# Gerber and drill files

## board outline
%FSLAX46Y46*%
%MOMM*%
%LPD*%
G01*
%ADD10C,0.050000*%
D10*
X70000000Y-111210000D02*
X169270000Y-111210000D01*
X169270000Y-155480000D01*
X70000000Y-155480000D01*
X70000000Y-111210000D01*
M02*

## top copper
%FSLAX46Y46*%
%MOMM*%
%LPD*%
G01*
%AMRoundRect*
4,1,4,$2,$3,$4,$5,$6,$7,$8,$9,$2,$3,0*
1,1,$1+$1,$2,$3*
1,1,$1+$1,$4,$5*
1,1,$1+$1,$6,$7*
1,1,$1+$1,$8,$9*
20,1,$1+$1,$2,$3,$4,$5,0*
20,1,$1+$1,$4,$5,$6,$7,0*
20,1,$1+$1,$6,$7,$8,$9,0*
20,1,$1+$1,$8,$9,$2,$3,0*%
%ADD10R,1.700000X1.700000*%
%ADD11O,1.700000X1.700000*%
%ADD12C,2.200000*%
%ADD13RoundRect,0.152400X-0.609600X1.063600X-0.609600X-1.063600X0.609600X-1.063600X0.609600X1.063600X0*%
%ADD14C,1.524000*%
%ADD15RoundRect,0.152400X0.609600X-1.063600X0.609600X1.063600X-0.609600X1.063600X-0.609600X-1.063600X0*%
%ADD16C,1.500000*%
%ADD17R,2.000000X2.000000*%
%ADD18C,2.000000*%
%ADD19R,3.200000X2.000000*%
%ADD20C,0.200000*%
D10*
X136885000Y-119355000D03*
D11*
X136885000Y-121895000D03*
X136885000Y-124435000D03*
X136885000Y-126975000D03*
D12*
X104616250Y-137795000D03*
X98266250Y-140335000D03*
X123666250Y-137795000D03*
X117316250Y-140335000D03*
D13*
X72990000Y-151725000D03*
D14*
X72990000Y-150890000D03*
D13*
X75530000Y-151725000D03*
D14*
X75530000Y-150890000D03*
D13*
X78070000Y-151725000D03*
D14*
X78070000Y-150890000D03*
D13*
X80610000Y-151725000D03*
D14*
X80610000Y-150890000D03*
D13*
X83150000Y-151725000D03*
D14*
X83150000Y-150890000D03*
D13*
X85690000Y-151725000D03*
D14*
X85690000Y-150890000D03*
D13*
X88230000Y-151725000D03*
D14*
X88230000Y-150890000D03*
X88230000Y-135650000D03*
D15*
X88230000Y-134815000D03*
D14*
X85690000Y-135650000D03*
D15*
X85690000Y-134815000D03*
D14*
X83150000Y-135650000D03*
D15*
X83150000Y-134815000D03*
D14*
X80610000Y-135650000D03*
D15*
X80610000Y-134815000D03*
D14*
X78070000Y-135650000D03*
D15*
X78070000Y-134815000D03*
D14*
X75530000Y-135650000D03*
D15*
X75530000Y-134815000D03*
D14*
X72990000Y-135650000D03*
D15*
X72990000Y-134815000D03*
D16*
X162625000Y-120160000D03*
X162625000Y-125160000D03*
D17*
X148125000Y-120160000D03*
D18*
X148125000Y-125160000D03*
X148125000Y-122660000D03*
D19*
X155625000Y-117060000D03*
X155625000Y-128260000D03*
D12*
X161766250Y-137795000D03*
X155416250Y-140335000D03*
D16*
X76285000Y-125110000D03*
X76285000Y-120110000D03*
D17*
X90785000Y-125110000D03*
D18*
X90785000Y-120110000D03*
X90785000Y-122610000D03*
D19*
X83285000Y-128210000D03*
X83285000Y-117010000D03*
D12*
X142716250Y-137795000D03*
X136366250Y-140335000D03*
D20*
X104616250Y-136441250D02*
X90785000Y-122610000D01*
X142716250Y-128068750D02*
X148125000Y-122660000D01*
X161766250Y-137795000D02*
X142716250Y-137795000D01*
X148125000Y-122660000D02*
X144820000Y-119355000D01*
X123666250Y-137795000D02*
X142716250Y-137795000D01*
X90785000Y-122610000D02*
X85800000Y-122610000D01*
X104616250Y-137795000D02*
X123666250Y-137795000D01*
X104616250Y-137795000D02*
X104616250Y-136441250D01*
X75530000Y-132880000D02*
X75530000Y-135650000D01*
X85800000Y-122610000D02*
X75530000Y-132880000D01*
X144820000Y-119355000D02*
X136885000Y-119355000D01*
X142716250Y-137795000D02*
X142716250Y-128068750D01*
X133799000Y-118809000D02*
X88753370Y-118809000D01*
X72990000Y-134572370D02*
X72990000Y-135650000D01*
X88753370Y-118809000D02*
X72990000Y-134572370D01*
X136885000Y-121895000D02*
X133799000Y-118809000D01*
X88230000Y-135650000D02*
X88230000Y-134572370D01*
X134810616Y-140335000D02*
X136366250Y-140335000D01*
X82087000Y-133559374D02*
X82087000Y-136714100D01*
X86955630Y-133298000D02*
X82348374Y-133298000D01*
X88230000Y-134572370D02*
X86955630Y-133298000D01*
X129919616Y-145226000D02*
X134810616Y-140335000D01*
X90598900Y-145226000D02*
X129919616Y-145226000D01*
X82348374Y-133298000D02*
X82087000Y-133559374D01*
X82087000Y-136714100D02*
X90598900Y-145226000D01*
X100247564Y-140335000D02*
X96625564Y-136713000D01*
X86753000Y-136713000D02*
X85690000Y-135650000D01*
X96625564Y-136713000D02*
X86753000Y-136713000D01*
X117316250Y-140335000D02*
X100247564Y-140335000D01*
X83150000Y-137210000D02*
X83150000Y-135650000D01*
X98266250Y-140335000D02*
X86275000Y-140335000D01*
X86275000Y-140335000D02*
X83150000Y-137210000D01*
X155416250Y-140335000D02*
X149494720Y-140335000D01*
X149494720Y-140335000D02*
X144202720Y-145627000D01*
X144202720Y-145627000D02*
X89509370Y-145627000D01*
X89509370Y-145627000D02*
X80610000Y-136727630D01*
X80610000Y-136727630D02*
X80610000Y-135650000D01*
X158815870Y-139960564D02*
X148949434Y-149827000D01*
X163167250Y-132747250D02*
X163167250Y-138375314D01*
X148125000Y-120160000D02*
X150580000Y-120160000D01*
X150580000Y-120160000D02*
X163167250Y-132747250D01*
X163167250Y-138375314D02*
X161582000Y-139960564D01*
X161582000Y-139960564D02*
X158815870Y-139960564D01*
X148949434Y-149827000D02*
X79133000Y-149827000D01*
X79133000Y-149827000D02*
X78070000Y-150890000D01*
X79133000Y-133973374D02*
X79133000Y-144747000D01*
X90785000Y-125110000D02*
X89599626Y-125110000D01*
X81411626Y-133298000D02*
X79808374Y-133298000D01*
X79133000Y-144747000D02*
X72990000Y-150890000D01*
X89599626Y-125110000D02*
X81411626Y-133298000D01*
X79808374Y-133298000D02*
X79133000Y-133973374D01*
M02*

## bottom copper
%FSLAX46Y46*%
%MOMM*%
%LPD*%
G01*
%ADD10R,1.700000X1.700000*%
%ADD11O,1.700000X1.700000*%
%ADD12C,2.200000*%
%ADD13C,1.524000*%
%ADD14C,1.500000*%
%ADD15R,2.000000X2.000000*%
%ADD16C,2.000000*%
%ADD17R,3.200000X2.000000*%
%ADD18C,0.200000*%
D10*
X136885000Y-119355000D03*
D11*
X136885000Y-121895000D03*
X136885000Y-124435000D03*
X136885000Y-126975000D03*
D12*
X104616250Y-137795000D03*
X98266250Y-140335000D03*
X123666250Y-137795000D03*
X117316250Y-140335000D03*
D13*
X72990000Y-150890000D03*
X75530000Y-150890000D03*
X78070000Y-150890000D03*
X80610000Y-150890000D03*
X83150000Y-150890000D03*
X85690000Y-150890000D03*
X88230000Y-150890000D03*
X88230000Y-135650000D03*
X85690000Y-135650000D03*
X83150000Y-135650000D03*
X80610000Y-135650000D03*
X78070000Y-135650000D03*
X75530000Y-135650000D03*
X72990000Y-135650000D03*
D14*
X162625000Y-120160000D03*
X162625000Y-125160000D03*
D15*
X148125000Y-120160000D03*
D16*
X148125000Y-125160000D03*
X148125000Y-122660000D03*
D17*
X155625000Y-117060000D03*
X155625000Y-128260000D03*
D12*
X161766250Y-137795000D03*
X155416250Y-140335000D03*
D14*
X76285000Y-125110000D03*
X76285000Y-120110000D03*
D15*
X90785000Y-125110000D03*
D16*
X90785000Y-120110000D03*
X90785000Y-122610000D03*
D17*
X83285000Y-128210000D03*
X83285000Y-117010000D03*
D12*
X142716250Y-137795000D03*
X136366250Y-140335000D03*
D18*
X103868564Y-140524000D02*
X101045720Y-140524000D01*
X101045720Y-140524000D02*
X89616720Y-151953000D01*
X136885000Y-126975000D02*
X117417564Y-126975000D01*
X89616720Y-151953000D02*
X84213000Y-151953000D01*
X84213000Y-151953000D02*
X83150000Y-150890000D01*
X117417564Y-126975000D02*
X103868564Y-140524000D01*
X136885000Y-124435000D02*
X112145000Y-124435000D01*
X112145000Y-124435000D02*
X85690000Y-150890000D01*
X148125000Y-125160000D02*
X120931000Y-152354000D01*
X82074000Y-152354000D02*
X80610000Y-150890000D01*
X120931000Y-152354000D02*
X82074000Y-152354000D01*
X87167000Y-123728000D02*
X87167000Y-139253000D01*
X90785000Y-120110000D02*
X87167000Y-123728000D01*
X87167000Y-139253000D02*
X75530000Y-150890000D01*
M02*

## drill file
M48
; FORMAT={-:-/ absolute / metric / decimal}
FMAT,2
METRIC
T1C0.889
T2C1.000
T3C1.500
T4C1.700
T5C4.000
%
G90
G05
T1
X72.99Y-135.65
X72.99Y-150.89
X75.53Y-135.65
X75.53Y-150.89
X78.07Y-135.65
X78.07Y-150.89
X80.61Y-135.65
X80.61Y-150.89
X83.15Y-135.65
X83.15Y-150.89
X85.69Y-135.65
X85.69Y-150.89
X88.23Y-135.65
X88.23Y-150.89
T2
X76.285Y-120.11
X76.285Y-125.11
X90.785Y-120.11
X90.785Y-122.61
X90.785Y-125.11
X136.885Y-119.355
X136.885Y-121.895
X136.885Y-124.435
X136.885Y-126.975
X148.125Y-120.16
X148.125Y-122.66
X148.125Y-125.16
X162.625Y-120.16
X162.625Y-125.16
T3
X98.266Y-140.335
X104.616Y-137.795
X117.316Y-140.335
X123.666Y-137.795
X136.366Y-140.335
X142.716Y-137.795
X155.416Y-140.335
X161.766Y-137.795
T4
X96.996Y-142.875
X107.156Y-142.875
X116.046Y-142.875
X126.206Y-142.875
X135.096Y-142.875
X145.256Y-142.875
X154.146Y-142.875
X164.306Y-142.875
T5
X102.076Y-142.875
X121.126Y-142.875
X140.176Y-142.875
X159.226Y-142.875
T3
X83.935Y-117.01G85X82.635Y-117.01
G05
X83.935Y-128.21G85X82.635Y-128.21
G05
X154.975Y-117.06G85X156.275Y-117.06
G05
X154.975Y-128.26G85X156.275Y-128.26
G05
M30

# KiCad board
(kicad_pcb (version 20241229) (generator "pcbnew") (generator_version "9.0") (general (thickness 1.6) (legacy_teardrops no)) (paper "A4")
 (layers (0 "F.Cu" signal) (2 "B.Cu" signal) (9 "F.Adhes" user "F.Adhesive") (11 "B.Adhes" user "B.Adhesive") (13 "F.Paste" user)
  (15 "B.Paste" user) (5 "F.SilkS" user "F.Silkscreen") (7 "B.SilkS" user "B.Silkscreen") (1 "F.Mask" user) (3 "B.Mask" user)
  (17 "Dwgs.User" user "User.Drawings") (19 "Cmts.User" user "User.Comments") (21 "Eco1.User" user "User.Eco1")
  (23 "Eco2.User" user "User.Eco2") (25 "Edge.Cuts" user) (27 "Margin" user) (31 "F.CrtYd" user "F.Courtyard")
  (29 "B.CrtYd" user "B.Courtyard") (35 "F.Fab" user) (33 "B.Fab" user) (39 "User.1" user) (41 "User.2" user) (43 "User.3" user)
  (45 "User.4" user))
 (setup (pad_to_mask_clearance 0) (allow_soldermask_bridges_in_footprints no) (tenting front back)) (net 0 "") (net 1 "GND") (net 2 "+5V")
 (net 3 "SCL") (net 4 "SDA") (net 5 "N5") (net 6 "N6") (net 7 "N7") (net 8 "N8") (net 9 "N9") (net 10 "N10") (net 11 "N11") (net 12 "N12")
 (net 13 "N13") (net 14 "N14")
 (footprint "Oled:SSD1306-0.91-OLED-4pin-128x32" (layer "F.Cu") (at 100.385 117.165)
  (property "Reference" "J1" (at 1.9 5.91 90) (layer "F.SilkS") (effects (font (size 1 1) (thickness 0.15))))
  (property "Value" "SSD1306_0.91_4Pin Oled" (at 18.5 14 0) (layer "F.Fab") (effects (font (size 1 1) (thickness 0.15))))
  (pad "1" thru_hole rect (at 36.5 2.19) (size 1.7 1.7) (drill 1) (layers "*.Cu" "*.Mask") (remove_unused_layers no) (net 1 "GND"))
  (pad "2" thru_hole oval (at 36.5 4.73) (size 1.7 1.7) (drill 1) (layers "*.Cu" "*.Mask") (remove_unused_layers no) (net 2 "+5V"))
  (pad "3" thru_hole oval (at 36.5 7.27) (size 1.7 1.7) (drill 1) (layers "*.Cu" "*.Mask") (remove_unused_layers no) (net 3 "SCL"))
  (pad "4" thru_hole oval (at 36.5 9.81) (size 1.7 1.7) (drill 1) (layers "*.Cu" "*.Mask") (remove_unused_layers no) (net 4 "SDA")))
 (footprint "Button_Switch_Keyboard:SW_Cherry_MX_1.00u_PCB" (layer "F.Cu") (at 104.61625 137.795)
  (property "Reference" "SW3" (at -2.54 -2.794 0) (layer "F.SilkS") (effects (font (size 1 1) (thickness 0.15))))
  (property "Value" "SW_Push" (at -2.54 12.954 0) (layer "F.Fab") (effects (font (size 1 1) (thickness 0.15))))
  (pad "" np_thru_hole circle (at -7.62 5.08) (size 1.7 1.7) (drill 1.7) (layers "*.Cu" "*.Mask"))
  (pad "" np_thru_hole circle (at -2.54 5.08) (size 4 4) (drill 4) (layers "*.Cu" "*.Mask"))
  (pad "" np_thru_hole circle (at 2.54 5.08) (size 1.7 1.7) (drill 1.7) (layers "*.Cu" "*.Mask"))
  (pad "1" thru_hole circle (at 0 0) (size 2.2 2.2) (drill 1.5) (layers "*.Cu" "*.Mask") (remove_unused_layers no) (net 1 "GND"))
  (pad "2" thru_hole circle (at -6.35 2.54) (size 2.2 2.2) (drill 1.5) (layers "*.Cu" "*.Mask") (remove_unused_layers no) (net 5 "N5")))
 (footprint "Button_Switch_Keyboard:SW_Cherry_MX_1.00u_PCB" (layer "F.Cu") (at 123.66625 137.795)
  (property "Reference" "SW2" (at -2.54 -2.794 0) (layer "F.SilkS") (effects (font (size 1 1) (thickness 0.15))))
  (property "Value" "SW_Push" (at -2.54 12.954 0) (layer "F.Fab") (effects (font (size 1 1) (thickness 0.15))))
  (pad "" np_thru_hole circle (at -7.62 5.08) (size 1.7 1.7) (drill 1.7) (layers "*.Cu" "*.Mask"))
  (pad "" np_thru_hole circle (at -2.54 5.08) (size 4 4) (drill 4) (layers "*.Cu" "*.Mask"))
  (pad "" np_thru_hole circle (at 2.54 5.08) (size 1.7 1.7) (drill 1.7) (layers "*.Cu" "*.Mask"))
  (pad "1" thru_hole circle (at 0 0) (size 2.2 2.2) (drill 1.5) (layers "*.Cu" "*.Mask") (remove_unused_layers no) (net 1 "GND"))
  (pad "2" thru_hole circle (at -6.35 2.54) (size 2.2 2.2) (drill 1.5) (layers "*.Cu" "*.Mask") (remove_unused_layers no) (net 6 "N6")))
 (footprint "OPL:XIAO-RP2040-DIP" (layer "F.Cu") (at 80.61 143.27 90)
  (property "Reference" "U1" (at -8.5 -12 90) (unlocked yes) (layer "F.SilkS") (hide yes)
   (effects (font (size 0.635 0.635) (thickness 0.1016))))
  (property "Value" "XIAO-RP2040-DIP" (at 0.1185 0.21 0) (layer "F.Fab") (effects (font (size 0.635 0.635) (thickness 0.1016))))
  (pad "1" smd roundrect (at -8.455 -7.62 270) (size 2.432 1.524) (layers "F.Cu" "F.Mask") (roundrect_rratio 0.1) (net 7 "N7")
   (thermal_bridge_angle 45))
  (pad "1" thru_hole circle (at -7.62 -7.62 270) (size 1.524 1.524) (drill 0.889) (layers "*.Cu" "*.Mask") (remove_unused_layers no)
   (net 7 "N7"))
  (pad "2" smd roundrect (at -8.455 -5.08 270) (size 2.432 1.524) (layers "F.Cu" "F.Mask") (roundrect_rratio 0.1) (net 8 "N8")
   (thermal_bridge_angle 45))
  (pad "2" thru_hole circle (at -7.62 -5.08 270) (size 1.524 1.524) (drill 0.889) (layers "*.Cu" "*.Mask") (remove_unused_layers no)
   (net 8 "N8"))
  (pad "3" smd roundrect (at -8.455 -2.54 270) (size 2.432 1.524) (layers "F.Cu" "F.Mask") (roundrect_rratio 0.1) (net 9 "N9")
   (thermal_bridge_angle 45))
  (pad "3" thru_hole circle (at -7.62 -2.54 270) (size 1.524 1.524) (drill 0.889) (layers "*.Cu" "*.Mask") (remove_unused_layers no)
   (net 9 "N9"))
  (pad "4" smd roundrect (at -8.455 0 270) (size 2.432 1.524) (layers "F.Cu" "F.Mask") (roundrect_rratio 0.1) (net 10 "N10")
   (thermal_bridge_angle 45))
  (pad "4" thru_hole circle (at -7.62 0 270) (size 1.524 1.524) (drill 0.889) (layers "*.Cu" "*.Mask") (remove_unused_layers no)
   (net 10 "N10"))
  (pad "5" smd roundrect (at -8.455 2.54 270) (size 2.432 1.524) (layers "F.Cu" "F.Mask") (roundrect_rratio 0.1) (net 4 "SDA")
   (thermal_bridge_angle 45))
  (pad "5" thru_hole circle (at -7.62 2.54 270) (size 1.524 1.524) (drill 0.889) (layers "*.Cu" "*.Mask") (remove_unused_layers no)
   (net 4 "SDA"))
  (pad "6" smd roundrect (at -8.455 5.08 270) (size 2.432 1.524) (layers "F.Cu" "F.Mask") (roundrect_rratio 0.1) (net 3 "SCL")
   (thermal_bridge_angle 45))
  (pad "6" thru_hole circle (at -7.62 5.08 270) (size 1.524 1.524) (drill 0.889) (layers "*.Cu" "*.Mask") (remove_unused_layers no)
   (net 3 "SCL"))
  (pad "7" smd roundrect (at -8.455 7.62 270) (size 2.432 1.524) (layers "F.Cu" "F.Mask") (roundrect_rratio 0.1) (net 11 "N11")
   (thermal_bridge_angle 45))
  (pad "7" thru_hole circle (at -7.62 7.62 270) (size 1.524 1.524) (drill 0.889) (layers "*.Cu" "*.Mask") (remove_unused_layers no)
   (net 11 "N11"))
  (pad "8" thru_hole circle (at 7.62 7.62 90) (size 1.524 1.524) (drill 0.889) (layers "*.Cu" "*.Mask") (remove_unused_layers no)
   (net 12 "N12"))
  (pad "8" smd roundrect (at 8.455 7.62 90) (size 2.432 1.524) (layers "F.Cu" "F.Mask") (roundrect_rratio 0.1) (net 12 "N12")
   (thermal_bridge_angle 45))
  (pad "9" thru_hole circle (at 7.62 5.08 90) (size 1.524 1.524) (drill 0.889) (layers "*.Cu" "*.Mask") (remove_unused_layers no)
   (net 6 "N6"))
  (pad "9" smd roundrect (at 8.455 5.08 90) (size 2.432 1.524) (layers "F.Cu" "F.Mask") (roundrect_rratio 0.1) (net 6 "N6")
   (thermal_bridge_angle 45))
  (pad "10" thru_hole circle (at 7.62 2.54 90) (size 1.524 1.524) (drill 0.889) (layers "*.Cu" "*.Mask") (remove_unused_layers no)
   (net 5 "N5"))
  (pad "10" smd roundrect (at 8.455 2.54 90) (size 2.432 1.524) (layers "F.Cu" "F.Mask") (roundrect_rratio 0.1) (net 5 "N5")
   (thermal_bridge_angle 45))
  (pad "11" thru_hole circle (at 7.62 0 90) (size 1.524 1.524) (drill 0.889) (layers "*.Cu" "*.Mask") (remove_unused_layers no)
   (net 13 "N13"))
  (pad "11" smd roundrect (at 8.455 0 90) (size 2.432 1.524) (layers "F.Cu" "F.Mask") (roundrect_rratio 0.1) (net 13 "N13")
   (thermal_bridge_angle 45))
  (pad "12" thru_hole circle (at 7.62 -2.54 90) (size 1.524 1.524) (drill 0.889) (layers "*.Cu" "*.Mask") (remove_unused_layers no)
   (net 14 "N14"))
  (pad "12" smd roundrect (at 8.455 -2.54 90) (size 2.432 1.524) (layers "F.Cu" "F.Mask") (roundrect_rratio 0.1) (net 14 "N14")
   (thermal_bridge_angle 45))
  (pad "13" thru_hole circle (at 7.62 -5.08 90) (size 1.524 1.524) (drill 0.889) (layers "*.Cu" "*.Mask") (remove_unused_layers no)
   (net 1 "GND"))
  (pad "13" smd roundrect (at 8.455 -5.08 90) (size 2.432 1.524) (layers "F.Cu" "F.Mask") (roundrect_rratio 0.1) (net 1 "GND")
   (thermal_bridge_angle 45))
  (pad "14" thru_hole circle (at 7.62 -7.62 90) (size 1.524 1.524) (drill 0.889) (layers "*.Cu" "*.Mask") (remove_unused_layers no)
   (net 2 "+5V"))
  (pad "14" smd roundrect (at 8.455 -7.62 90) (size 2.432 1.524) (layers "F.Cu" "F.Mask") (roundrect_rratio 0.1) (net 2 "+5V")
   (thermal_bridge_angle 45)))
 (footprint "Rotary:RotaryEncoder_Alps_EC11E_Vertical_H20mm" (layer "F.Cu") (at 148.125 120.16)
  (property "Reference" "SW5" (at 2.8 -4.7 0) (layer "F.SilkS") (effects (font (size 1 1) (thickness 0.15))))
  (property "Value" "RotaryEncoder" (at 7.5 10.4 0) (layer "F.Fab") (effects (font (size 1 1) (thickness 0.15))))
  (pad "" thru_hole circle (at 14.5 0) (size 1.5 1.5) (drill 1) (layers "*.Cu" "*.Mask") (remove_unused_layers no))
  (pad "" thru_hole circle (at 14.5 5) (size 1.5 1.5) (drill 1) (layers "*.Cu" "*.Mask") (remove_unused_layers no))
  (pad "A" thru_hole rect (at 0 0) (size 2 2) (drill 1) (layers "*.Cu" "*.Mask") (remove_unused_layers no) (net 9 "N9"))
  (pad "B" thru_hole circle (at 0 5) (size 2 2) (drill 1) (layers "*.Cu" "*.Mask") (remove_unused_layers no) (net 10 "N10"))
  (pad "C" thru_hole circle (at 0 2.5) (size 2 2) (drill 1) (layers "*.Cu" "*.Mask") (remove_unused_layers no) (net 1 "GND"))
  (pad "MP" thru_hole rect (at 7.5 -3.1) (size 3.2 2) (drill oval 2.8 1.5) (layers "*.Cu" "*.Mask") (remove_unused_layers no))
  (pad "MP" thru_hole rect (at 7.5 8.1) (size 3.2 2) (drill oval 2.8 1.5) (layers "*.Cu" "*.Mask") (remove_unused_layers no)))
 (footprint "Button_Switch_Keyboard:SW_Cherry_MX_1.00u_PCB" (layer "F.Cu") (at 161.76625 137.795)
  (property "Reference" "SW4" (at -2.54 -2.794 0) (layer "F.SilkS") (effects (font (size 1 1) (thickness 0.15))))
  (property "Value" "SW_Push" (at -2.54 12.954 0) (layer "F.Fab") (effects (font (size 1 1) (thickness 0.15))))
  (pad "" np_thru_hole circle (at -7.62 5.08) (size 1.7 1.7) (drill 1.7) (layers "*.Cu" "*.Mask"))
  (pad "" np_thru_hole circle (at -2.54 5.08) (size 4 4) (drill 4) (layers "*.Cu" "*.Mask"))
  (pad "" np_thru_hole circle (at 2.54 5.08) (size 1.7 1.7) (drill 1.7) (layers "*.Cu" "*.Mask"))
  (pad "1" thru_hole circle (at 0 0) (size 2.2 2.2) (drill 1.5) (layers "*.Cu" "*.Mask") (remove_unused_layers no) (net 1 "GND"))
  (pad "2" thru_hole circle (at -6.35 2.54) (size 2.2 2.2) (drill 1.5) (layers "*.Cu" "*.Mask") (remove_unused_layers no) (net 13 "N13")))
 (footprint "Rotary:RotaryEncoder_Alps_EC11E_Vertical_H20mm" (layer "F.Cu") (at 90.785 125.11 180)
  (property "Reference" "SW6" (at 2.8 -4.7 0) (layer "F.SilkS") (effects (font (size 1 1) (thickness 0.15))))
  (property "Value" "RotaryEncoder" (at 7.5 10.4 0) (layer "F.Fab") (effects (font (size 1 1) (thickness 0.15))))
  (pad "" thru_hole circle (at 14.5 0 180) (size 1.5 1.5) (drill 1) (layers "*.Cu" "*.Mask") (remove_unused_layers no))
  (pad "" thru_hole circle (at 14.5 5 180) (size 1.5 1.5) (drill 1) (layers "*.Cu" "*.Mask") (remove_unused_layers no))
  (pad "A" thru_hole rect (at 0 0 180) (size 2 2) (drill 1) (layers "*.Cu" "*.Mask") (remove_unused_layers no) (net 7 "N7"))
  (pad "B" thru_hole circle (at 0 5 180) (size 2 2) (drill 1) (layers "*.Cu" "*.Mask") (remove_unused_layers no) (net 8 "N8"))
  (pad "C" thru_hole circle (at 0 2.5 180) (size 2 2) (drill 1) (layers "*.Cu" "*.Mask") (remove_unused_layers no) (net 1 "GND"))
  (pad "MP" thru_hole rect (at 7.5 -3.1 180) (size 3.2 2) (drill oval 2.8 1.5) (layers "*.Cu" "*.Mask") (remove_unused_layers no))
  (pad "MP" thru_hole rect (at 7.5 8.1 180) (size 3.2 2) (drill oval 2.8 1.5) (layers "*.Cu" "*.Mask") (remove_unused_layers no)))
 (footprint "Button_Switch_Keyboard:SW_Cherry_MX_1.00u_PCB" (layer "F.Cu") (at 142.71625 137.795)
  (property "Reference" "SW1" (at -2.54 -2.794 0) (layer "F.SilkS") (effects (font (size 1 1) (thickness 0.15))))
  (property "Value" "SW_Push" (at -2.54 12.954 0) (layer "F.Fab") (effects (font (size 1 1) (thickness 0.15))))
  (pad "" np_thru_hole circle (at -7.62 5.08) (size 1.7 1.7) (drill 1.7) (layers "*.Cu" "*.Mask"))
  (pad "" np_thru_hole circle (at -2.54 5.08) (size 4 4) (drill 4) (layers "*.Cu" "*.Mask"))
  (pad "" np_thru_hole circle (at 2.54 5.08) (size 1.7 1.7) (drill 1.7) (layers "*.Cu" "*.Mask"))
  (pad "1" thru_hole circle (at 0 0) (size 2.2 2.2) (drill 1.5) (layers "*.Cu" "*.Mask") (remove_unused_layers no) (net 1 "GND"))
  (pad "2" thru_hole circle (at -6.35 2.54) (size 2.2 2.2) (drill 1.5) (layers "*.Cu" "*.Mask") (remove_unused_layers no) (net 12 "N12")))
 (gr_rect (start 70 111.21) (end 169.27 155.48) (stroke (width 0.05) (type default)) (fill no) (layer "Edge.Cuts"))
 (segment (start 103.868564 140.524) (end 101.04572 140.524) (width 0.2) (layer "B.Cu") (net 4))
 (segment (start 101.04572 140.524) (end 89.61672 151.953) (width 0.2) (layer "B.Cu") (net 4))
 (segment (start 136.885 126.975) (end 117.417564 126.975) (width 0.2) (layer "B.Cu") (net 4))
 (segment (start 89.61672 151.953) (end 84.213 151.953) (width 0.2) (layer "B.Cu") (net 4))
 (segment (start 84.213 151.953) (end 83.15 150.89) (width 0.2) (layer "B.Cu") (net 4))
 (segment (start 117.417564 126.975) (end 103.868564 140.524) (width 0.2) (layer "B.Cu") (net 4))
 (segment (start 104.61625 136.44125) (end 90.785 122.61) (width 0.2) (layer "F.Cu") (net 1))
 (segment (start 142.71625 128.06875) (end 148.125 122.66) (width 0.2) (layer "F.Cu") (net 1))
 (segment (start 161.76625 137.795) (end 142.71625 137.795) (width 0.2) (layer "F.Cu") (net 1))
 (segment (start 148.125 122.66) (end 144.82 119.355) (width 0.2) (layer "F.Cu") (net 1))
 (segment (start 123.66625 137.795) (end 142.71625 137.795) (width 0.2) (layer "F.Cu") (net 1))
 (segment (start 90.785 122.61) (end 85.8 122.61) (width 0.2) (layer "F.Cu") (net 1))
 (segment (start 104.61625 137.795) (end 123.66625 137.795) (width 0.2) (layer "F.Cu") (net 1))
 (segment (start 104.61625 137.795) (end 104.61625 136.44125) (width 0.2) (layer "F.Cu") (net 1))
 (segment (start 75.53 132.88) (end 75.53 135.65) (width 0.2) (layer "F.Cu") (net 1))
 (segment (start 85.8 122.61) (end 75.53 132.88) (width 0.2) (layer "F.Cu") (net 1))
 (segment (start 144.82 119.355) (end 136.885 119.355) (width 0.2) (layer "F.Cu") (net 1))
 (segment (start 142.71625 137.795) (end 142.71625 128.06875) (width 0.2) (layer "F.Cu") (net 1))
 (segment (start 133.799 118.809) (end 88.75337 118.809) (width 0.2) (layer "F.Cu") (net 2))
 (segment (start 72.99 134.57237) (end 72.99 135.65) (width 0.2) (layer "F.Cu") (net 2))
 (segment (start 88.75337 118.809) (end 72.99 134.57237) (width 0.2) (layer "F.Cu") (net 2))
 (segment (start 136.885 121.895) (end 133.799 118.809) (width 0.2) (layer "F.Cu") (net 2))
 (segment (start 136.885 124.435) (end 112.145 124.435) (width 0.2) (layer "B.Cu") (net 3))
 (segment (start 112.145 124.435) (end 85.69 150.89) (width 0.2) (layer "B.Cu") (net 3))
 (segment (start 88.23 135.65) (end 88.23 134.57237) (width 0.2) (layer "F.Cu") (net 12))
 (segment (start 134.810616 140.335) (end 136.36625 140.335) (width 0.2) (layer "F.Cu") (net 12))
 (segment (start 82.087 133.559374) (end 82.087 136.7141) (width 0.2) (layer "F.Cu") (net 12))
 (segment (start 86.95563 133.298) (end 82.348374 133.298) (width 0.2) (layer "F.Cu") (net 12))
 (segment (start 88.23 134.57237) (end 86.95563 133.298) (width 0.2) (layer "F.Cu") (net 12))
 (segment (start 129.919616 145.226) (end 134.810616 140.335) (width 0.2) (layer "F.Cu") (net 12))
 (segment (start 90.5989 145.226) (end 129.919616 145.226) (width 0.2) (layer "F.Cu") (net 12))
 (segment (start 82.348374 133.298) (end 82.087 133.559374) (width 0.2) (layer "F.Cu") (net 12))
 (segment (start 82.087 136.7141) (end 90.5989 145.226) (width 0.2) (layer "F.Cu") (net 12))
 (segment (start 100.247564 140.335) (end 96.625564 136.713) (width 0.2) (layer "F.Cu") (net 6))
 (segment (start 86.753 136.713) (end 85.69 135.65) (width 0.2) (layer "F.Cu") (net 6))
 (segment (start 96.625564 136.713) (end 86.753 136.713) (width 0.2) (layer "F.Cu") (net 6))
 (segment (start 117.31625 140.335) (end 100.247564 140.335) (width 0.2) (layer "F.Cu") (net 6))
 (segment (start 83.15 137.21) (end 83.15 135.65) (width 0.2) (layer "F.Cu") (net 5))
 (segment (start 98.26625 140.335) (end 86.275 140.335) (width 0.2) (layer "F.Cu") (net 5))
 (segment (start 86.275 140.335) (end 83.15 137.21) (width 0.2) (layer "F.Cu") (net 5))
 (segment (start 155.41625 140.335) (end 149.49472 140.335) (width 0.2) (layer "F.Cu") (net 13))
 (segment (start 149.49472 140.335) (end 144.20272 145.627) (width 0.2) (layer "F.Cu") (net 13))
 (segment (start 144.20272 145.627) (end 89.50937 145.627) (width 0.2) (layer "F.Cu") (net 13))
 (segment (start 89.50937 145.627) (end 80.61 136.72763) (width 0.2) (layer "F.Cu") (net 13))
 (segment (start 80.61 136.72763) (end 80.61 135.65) (width 0.2) (layer "F.Cu") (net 13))
 (segment (start 148.125 125.16) (end 120.931 152.354) (width 0.2) (layer "B.Cu") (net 10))
 (segment (start 82.074 152.354) (end 80.61 150.89) (width 0.2) (layer "B.Cu") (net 10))
 (segment (start 120.931 152.354) (end 82.074 152.354) (width 0.2) (layer "B.Cu") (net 10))
 (segment (start 158.81587 139.960564) (end 148.949434 149.827) (width 0.2) (layer "F.Cu") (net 9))
 (segment (start 163.16725 132.74725) (end 163.16725 138.375314) (width 0.2) (layer "F.Cu") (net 9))
 (segment (start 148.125 120.16) (end 150.58 120.16) (width 0.2) (layer "F.Cu") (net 9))
 (segment (start 150.58 120.16) (end 163.16725 132.74725) (width 0.2) (layer "F.Cu") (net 9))
 (segment (start 163.16725 138.375314) (end 161.582 139.960564) (width 0.2) (layer "F.Cu") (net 9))
 (segment (start 161.582 139.960564) (end 158.81587 139.960564) (width 0.2) (layer "F.Cu") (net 9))
 (segment (start 148.949434 149.827) (end 79.133 149.827) (width 0.2) (layer "F.Cu") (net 9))
 (segment (start 79.133 149.827) (end 78.07 150.89) (width 0.2) (layer "F.Cu") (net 9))
 (segment (start 79.133 133.973374) (end 79.133 144.747) (width 0.2) (layer "F.Cu") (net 7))
 (segment (start 90.785 125.11) (end 89.599626 125.11) (width 0.2) (layer "F.Cu") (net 7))
 (segment (start 81.411626 133.298) (end 79.808374 133.298) (width 0.2) (layer "F.Cu") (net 7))
 (segment (start 79.133 144.747) (end 72.99 150.89) (width 0.2) (layer "F.Cu") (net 7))
 (segment (start 89.599626 125.11) (end 81.411626 133.298) (width 0.2) (layer "F.Cu") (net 7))
 (segment (start 79.808374 133.298) (end 79.133 133.973374) (width 0.2) (layer "F.Cu") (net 7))
 (segment (start 87.167 123.728) (end 87.167 139.253) (width 0.2) (layer "B.Cu") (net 8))
 (segment (start 90.785 120.11) (end 87.167 123.728) (width 0.2) (layer "B.Cu") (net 8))
 (segment (start 87.167 139.253) (end 75.53 150.89) (width 0.2) (layer "B.Cu") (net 8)))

